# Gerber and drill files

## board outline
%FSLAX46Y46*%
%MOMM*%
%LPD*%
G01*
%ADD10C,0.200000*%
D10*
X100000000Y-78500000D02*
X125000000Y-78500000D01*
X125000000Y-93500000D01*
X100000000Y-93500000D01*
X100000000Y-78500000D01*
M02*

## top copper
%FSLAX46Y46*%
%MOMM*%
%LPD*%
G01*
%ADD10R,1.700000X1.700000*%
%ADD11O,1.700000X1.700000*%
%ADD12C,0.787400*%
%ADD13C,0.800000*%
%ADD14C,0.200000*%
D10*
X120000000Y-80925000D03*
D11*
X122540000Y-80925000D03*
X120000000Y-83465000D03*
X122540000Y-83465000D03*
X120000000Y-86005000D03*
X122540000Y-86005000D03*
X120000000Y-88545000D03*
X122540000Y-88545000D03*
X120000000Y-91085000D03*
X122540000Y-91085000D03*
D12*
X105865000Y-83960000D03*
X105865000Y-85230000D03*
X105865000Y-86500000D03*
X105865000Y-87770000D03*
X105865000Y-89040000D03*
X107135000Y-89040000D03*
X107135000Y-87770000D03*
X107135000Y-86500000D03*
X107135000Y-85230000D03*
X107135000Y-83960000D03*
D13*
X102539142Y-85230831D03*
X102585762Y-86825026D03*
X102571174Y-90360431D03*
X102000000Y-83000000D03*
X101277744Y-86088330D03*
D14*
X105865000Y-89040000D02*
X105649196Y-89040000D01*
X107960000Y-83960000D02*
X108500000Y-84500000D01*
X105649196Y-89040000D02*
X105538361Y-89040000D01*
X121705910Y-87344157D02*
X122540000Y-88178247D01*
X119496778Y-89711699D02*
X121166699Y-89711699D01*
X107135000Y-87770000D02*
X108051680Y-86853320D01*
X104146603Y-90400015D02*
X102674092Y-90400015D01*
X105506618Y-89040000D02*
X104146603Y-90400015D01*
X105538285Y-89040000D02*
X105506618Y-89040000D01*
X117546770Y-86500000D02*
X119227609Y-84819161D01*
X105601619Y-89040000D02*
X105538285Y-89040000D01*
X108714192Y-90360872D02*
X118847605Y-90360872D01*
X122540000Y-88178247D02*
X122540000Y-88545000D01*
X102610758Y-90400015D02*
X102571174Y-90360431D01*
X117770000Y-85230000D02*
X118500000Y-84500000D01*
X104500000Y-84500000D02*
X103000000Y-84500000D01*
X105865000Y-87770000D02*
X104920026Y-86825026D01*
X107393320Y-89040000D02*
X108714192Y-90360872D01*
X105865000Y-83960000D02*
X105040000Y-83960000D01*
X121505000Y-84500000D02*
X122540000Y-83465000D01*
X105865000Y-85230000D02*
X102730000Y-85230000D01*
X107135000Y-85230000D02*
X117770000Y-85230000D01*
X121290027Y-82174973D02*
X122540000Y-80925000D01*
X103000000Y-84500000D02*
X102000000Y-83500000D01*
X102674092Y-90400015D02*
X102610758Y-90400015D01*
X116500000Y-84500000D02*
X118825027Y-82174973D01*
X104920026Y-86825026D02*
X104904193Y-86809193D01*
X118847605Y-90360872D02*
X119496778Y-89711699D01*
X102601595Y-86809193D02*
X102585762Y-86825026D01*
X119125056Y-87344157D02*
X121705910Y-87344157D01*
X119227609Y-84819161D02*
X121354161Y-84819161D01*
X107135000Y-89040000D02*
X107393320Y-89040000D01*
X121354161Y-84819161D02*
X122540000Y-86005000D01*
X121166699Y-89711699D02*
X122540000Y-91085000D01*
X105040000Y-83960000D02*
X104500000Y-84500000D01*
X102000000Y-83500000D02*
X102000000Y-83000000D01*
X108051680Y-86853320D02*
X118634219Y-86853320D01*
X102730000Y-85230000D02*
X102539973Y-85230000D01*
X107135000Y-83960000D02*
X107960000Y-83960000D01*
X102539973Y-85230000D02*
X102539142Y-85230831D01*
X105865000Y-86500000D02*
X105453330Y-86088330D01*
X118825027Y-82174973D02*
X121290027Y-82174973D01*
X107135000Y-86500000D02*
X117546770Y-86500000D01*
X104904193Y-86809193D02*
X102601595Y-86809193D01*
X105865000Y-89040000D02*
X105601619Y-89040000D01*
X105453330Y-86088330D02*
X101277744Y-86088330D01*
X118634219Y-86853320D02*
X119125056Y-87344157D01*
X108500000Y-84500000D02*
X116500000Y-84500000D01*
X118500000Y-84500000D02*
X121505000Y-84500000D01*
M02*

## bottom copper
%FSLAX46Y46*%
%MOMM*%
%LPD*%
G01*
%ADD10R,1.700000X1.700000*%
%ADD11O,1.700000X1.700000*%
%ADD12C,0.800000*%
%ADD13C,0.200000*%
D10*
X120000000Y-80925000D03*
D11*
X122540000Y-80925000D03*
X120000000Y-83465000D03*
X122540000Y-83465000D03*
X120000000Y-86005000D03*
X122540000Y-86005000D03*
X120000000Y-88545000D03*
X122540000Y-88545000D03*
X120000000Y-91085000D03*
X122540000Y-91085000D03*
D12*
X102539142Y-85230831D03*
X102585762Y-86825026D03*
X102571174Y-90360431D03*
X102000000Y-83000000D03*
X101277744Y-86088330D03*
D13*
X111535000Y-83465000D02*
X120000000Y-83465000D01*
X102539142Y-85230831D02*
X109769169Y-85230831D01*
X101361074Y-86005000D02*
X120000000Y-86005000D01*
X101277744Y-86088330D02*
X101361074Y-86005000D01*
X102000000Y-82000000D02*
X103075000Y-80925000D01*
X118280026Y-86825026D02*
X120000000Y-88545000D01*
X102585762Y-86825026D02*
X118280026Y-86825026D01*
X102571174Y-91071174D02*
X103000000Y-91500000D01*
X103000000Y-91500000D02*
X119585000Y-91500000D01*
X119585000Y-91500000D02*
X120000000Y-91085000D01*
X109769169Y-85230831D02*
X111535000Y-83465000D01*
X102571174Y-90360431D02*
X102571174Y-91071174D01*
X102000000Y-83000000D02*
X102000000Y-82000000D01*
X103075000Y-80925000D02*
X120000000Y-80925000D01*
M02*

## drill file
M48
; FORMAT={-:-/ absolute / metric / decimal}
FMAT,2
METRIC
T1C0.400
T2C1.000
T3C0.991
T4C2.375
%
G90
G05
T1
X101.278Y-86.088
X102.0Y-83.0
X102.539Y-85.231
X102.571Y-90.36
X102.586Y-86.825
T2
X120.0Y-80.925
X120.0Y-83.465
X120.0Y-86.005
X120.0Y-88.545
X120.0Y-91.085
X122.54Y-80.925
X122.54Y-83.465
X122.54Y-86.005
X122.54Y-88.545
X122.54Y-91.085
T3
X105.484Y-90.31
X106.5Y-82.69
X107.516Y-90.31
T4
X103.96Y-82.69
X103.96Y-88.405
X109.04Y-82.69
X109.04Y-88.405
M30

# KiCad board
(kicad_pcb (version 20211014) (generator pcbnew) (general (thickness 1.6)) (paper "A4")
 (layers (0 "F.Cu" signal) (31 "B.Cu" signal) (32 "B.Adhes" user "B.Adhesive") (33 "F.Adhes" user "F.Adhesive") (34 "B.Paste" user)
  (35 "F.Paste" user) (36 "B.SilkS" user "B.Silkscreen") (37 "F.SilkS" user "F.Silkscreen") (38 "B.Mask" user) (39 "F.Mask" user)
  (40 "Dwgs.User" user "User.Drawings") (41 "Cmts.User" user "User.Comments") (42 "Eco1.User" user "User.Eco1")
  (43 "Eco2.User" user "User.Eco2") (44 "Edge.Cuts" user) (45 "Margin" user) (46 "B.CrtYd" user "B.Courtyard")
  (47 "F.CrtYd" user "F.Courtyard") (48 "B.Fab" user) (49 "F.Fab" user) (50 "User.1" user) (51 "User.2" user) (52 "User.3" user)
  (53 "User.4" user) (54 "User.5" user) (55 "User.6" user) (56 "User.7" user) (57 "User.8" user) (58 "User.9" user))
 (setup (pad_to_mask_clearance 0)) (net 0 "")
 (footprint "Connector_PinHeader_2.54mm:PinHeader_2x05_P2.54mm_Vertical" (layer "F.Cu") (at 120 80.925)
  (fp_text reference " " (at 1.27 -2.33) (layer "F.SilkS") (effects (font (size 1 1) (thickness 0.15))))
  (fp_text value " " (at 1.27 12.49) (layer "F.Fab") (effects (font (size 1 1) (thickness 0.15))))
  (pad "1" thru_hole rect (at 0 0) (size 1.7 1.7) (drill 1) (layers *.Cu *.Mask))
  (pad "2" thru_hole oval (at 2.54 0) (size 1.7 1.7) (drill 1) (layers *.Cu *.Mask))
  (pad "3" thru_hole oval (at 0 2.54) (size 1.7 1.7) (drill 1) (layers *.Cu *.Mask))
  (pad "4" thru_hole oval (at 2.54 2.54) (size 1.7 1.7) (drill 1) (layers *.Cu *.Mask))
  (pad "5" thru_hole oval (at 0 5.08) (size 1.7 1.7) (drill 1) (layers *.Cu *.Mask))
  (pad "6" thru_hole oval (at 2.54 5.08) (size 1.7 1.7) (drill 1) (layers *.Cu *.Mask))
  (pad "7" thru_hole oval (at 0 7.62) (size 1.7 1.7) (drill 1) (layers *.Cu *.Mask))
  (pad "8" thru_hole oval (at 2.54 7.62) (size 1.7 1.7) (drill 1) (layers *.Cu *.Mask))
  (pad "9" thru_hole oval (at 0 10.16) (size 1.7 1.7) (drill 1) (layers *.Cu *.Mask))
  (pad "10" thru_hole oval (at 2.54 10.16) (size 1.7 1.7) (drill 1) (layers *.Cu *.Mask)))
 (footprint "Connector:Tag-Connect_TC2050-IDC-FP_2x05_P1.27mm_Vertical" (layer "F.Cu") (at 106.5 86.5 -90)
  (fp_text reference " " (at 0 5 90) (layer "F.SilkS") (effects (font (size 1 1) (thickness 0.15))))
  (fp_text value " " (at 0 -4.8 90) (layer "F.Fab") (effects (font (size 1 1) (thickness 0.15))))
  (pad "" np_thru_hole circle (at -3.81 0 270) (size 0.9906 0.9906) (drill 0.9906) (layers *.Cu *.Mask))
  (pad "" np_thru_hole circle (at 3.81 -1.016 270) (size 0.9906 0.9906) (drill 0.9906) (layers *.Cu *.Mask))
  (pad "" np_thru_hole circle (at 1.905 2.54 270) (size 2.3749 2.3749) (drill 2.3749) (layers *.Cu *.Mask))
  (pad "" np_thru_hole circle (at -3.81 2.54 270) (size 2.3749 2.3749) (drill 2.3749) (layers *.Cu *.Mask))
  (pad "" np_thru_hole circle (at -3.81 -2.54 270) (size 2.3749 2.3749) (drill 2.3749) (layers *.Cu *.Mask))
  (pad "" np_thru_hole circle (at 1.905 -2.54 270) (size 2.3749 2.3749) (drill 2.3749) (layers *.Cu *.Mask))
  (pad "" np_thru_hole circle (at 3.81 1.016 270) (size 0.9906 0.9906) (drill 0.9906) (layers *.Cu *.Mask))
  (pad "1" connect circle (at -2.54 0.635 270) (size 0.7874 0.7874) (layers "F.Cu" "F.Mask"))
  (pad "2" connect circle (at -1.27 0.635 270) (size 0.7874 0.7874) (layers "F.Cu" "F.Mask"))
  (pad "3" connect circle (at 0 0.635 270) (size 0.7874 0.7874) (layers "F.Cu" "F.Mask"))
  (pad "4" connect circle (at 1.27 0.635 270) (size 0.7874 0.7874) (layers "F.Cu" "F.Mask"))
  (pad "5" connect circle (at 2.54 0.635 270) (size 0.7874 0.7874) (layers "F.Cu" "F.Mask"))
  (pad "6" connect circle (at 2.54 -0.635 270) (size 0.7874 0.7874) (layers "F.Cu" "F.Mask"))
  (pad "7" connect circle (at 1.27 -0.635 270) (size 0.7874 0.7874) (layers "F.Cu" "F.Mask"))
  (pad "8" connect circle (at 0 -0.635 270) (size 0.7874 0.7874) (layers "F.Cu" "F.Mask"))
  (pad "9" connect circle (at -1.27 -0.635 270) (size 0.7874 0.7874) (layers "F.Cu" "F.Mask"))
  (pad "10" connect circle (at -2.54 -0.635 270) (size 0.7874 0.7874) (layers "F.Cu" "F.Mask")))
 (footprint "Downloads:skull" (layer "B.Cu") (at 114.5 86 180)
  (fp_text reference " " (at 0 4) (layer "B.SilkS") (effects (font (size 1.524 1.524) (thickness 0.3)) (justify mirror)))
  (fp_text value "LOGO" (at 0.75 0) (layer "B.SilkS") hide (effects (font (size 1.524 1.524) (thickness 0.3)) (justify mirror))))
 (gr_rect (start 100 78.5) (end 125 93.5) (layer "Edge.Cuts") (width 0.2) (fill none))
 (segment (start 105.865 89.04) (end 105.649196 89.04) (width 0.2) (layer "F.Cu") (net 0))
 (segment (start 107.96 83.96) (end 108.5 84.5) (width 0.2) (layer "F.Cu") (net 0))
 (segment (start 105.649196 89.04) (end 105.538361 89.04) (width 0.2) (layer "F.Cu") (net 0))
 (segment (start 121.70591 87.344157) (end 122.54 88.178247) (width 0.2) (layer "F.Cu") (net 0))
 (segment (start 119.496778 89.711699) (end 121.166699 89.711699) (width 0.2) (layer "F.Cu") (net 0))
 (segment (start 107.135 87.77) (end 108.05168 86.85332) (width 0.2) (layer "F.Cu") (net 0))
 (segment (start 104.146603 90.400015) (end 102.674092 90.400015) (width 0.2) (layer "F.Cu") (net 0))
 (segment (start 105.506618 89.04) (end 104.146603 90.400015) (width 0.2) (layer "F.Cu") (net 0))
 (segment (start 105.538285 89.04) (end 105.506618 89.04) (width 0.2) (layer "F.Cu") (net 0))
 (segment (start 117.54677 86.5) (end 119.227609 84.819161) (width 0.2) (layer "F.Cu") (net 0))
 (segment (start 105.601619 89.04) (end 105.538285 89.04) (width 0.2) (layer "F.Cu") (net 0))
 (segment (start 108.714192 90.360872) (end 118.847605 90.360872) (width 0.2) (layer "F.Cu") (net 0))
 (segment (start 122.54 88.178247) (end 122.54 88.545) (width 0.2) (layer "F.Cu") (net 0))
 (segment (start 102.610758 90.400015) (end 102.571174 90.360431) (width 0.2) (layer "F.Cu") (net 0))
 (segment (start 117.77 85.23) (end 118.5 84.5) (width 0.2) (layer "F.Cu") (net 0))
 (segment (start 104.5 84.5) (end 103 84.5) (width 0.2) (layer "F.Cu") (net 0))
 (segment (start 105.865 87.77) (end 104.920026 86.825026) (width 0.2) (layer "F.Cu") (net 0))
 (segment (start 107.39332 89.04) (end 108.714192 90.360872) (width 0.2) (layer "F.Cu") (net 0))
 (segment (start 105.865 83.96) (end 105.04 83.96) (width 0.2) (layer "F.Cu") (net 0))
 (segment (start 121.505 84.5) (end 122.54 83.465) (width 0.2) (layer "F.Cu") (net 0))
 (segment (start 105.865 85.23) (end 102.73 85.23) (width 0.2) (layer "F.Cu") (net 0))
 (segment (start 107.135 85.23) (end 117.77 85.23) (width 0.2) (layer "F.Cu") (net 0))
 (segment (start 121.290027 82.174973) (end 122.54 80.925) (width 0.2) (layer "F.Cu") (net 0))
 (segment (start 103 84.5) (end 102 83.5) (width 0.2) (layer "F.Cu") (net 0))
 (segment (start 102.674092 90.400015) (end 102.610758 90.400015) (width 0.2) (layer "F.Cu") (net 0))
 (segment (start 116.5 84.5) (end 118.825027 82.174973) (width 0.2) (layer "F.Cu") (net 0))
 (segment (start 104.920026 86.825026) (end 104.904193 86.809193) (width 0.2) (layer "F.Cu") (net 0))
 (segment (start 118.847605 90.360872) (end 119.496778 89.711699) (width 0.2) (layer "F.Cu") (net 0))
 (segment (start 102.601595 86.809193) (end 102.585762 86.825026) (width 0.2) (layer "F.Cu") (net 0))
 (segment (start 119.125056 87.344157) (end 121.70591 87.344157) (width 0.2) (layer "F.Cu") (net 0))
 (segment (start 119.227609 84.819161) (end 121.354161 84.819161) (width 0.2) (layer "F.Cu") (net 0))
 (segment (start 107.135 89.04) (end 107.39332 89.04) (width 0.2) (layer "F.Cu") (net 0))
 (segment (start 121.354161 84.819161) (end 122.54 86.005) (width 0.2) (layer "F.Cu") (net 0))
 (segment (start 121.166699 89.711699) (end 122.54 91.085) (width 0.2) (layer "F.Cu") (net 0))
 (segment (start 105.04 83.96) (end 104.5 84.5) (width 0.2) (layer "F.Cu") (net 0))
 (segment (start 102 83.5) (end 102 83) (width 0.2) (layer "F.Cu") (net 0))
 (segment (start 108.05168 86.85332) (end 118.634219 86.85332) (width 0.2) (layer "F.Cu") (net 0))
 (segment (start 102.73 85.23) (end 102.539973 85.23) (width 0.2) (layer "F.Cu") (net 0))
 (segment (start 107.135 83.96) (end 107.96 83.96) (width 0.2) (layer "F.Cu") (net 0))
 (segment (start 102.539973 85.23) (end 102.539142 85.230831) (width 0.2) (layer "F.Cu") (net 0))
 (segment (start 105.865 86.5) (end 105.45333 86.08833) (width 0.2) (layer "F.Cu") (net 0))
 (segment (start 118.825027 82.174973) (end 121.290027 82.174973) (width 0.2) (layer "F.Cu") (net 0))
 (segment (start 107.135 86.5) (end 117.54677 86.5) (width 0.2) (layer "F.Cu") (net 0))
 (segment (start 104.904193 86.809193) (end 102.601595 86.809193) (width 0.2) (layer "F.Cu") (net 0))
 (segment (start 105.865 89.04) (end 105.601619 89.04) (width 0.2) (layer "F.Cu") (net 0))
 (segment (start 105.45333 86.08833) (end 101.277744 86.08833) (width 0.2) (layer "F.Cu") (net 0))
 (segment (start 118.634219 86.85332) (end 119.125056 87.344157) (width 0.2) (layer "F.Cu") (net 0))
 (segment (start 108.5 84.5) (end 116.5 84.5) (width 0.2) (layer "F.Cu") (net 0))
 (segment (start 118.5 84.5) (end 121.505 84.5) (width 0.2) (layer "F.Cu") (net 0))
 (via (at 102.539142 85.230831) (size 0.8) (drill 0.4) (layers "F.Cu" "B.Cu") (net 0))
 (via (at 102.585762 86.825026) (size 0.8) (drill 0.4) (layers "F.Cu" "B.Cu") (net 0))
 (via (at 102.571174 90.360431) (size 0.8) (drill 0.4) (layers "F.Cu" "B.Cu") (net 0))
 (via (at 102 83) (size 0.8) (drill 0.4) (layers "F.Cu" "B.Cu") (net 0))
 (via (at 101.277744 86.08833) (size 0.8) (drill 0.4) (layers "F.Cu" "B.Cu") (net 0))
 (segment (start 111.535 83.465) (end 120 83.465) (width 0.2) (layer "B.Cu") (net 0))
 (segment (start 102.539142 85.230831) (end 109.769169 85.230831) (width 0.2) (layer "B.Cu") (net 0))
 (segment (start 101.361074 86.005) (end 120 86.005) (width 0.2) (layer "B.Cu") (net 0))
 (segment (start 101.277744 86.08833) (end 101.361074 86.005) (width 0.2) (layer "B.Cu") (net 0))
 (segment (start 102 82) (end 103.075 80.925) (width 0.2) (layer "B.Cu") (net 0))
 (segment (start 118.280026 86.825026) (end 120 88.545) (width 0.2) (layer "B.Cu") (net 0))
 (segment (start 102.585762 86.825026) (end 118.280026 86.825026) (width 0.2) (layer "B.Cu") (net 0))
 (segment (start 102.571174 91.071174) (end 103 91.5) (width 0.2) (layer "B.Cu") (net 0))
 (segment (start 103 91.5) (end 119.585 91.5) (width 0.2) (layer "B.Cu") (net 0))
 (segment (start 119.585 91.5) (end 120 91.085) (width 0.2) (layer "B.Cu") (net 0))
 (segment (start 109.769169 85.230831) (end 111.535 83.465) (width 0.2) (layer "B.Cu") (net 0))
 (segment (start 102.571174 90.360431) (end 102.571174 91.071174) (width 0.2) (layer "B.Cu") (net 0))
 (segment (start 102 83) (end 102 82) (width 0.2) (layer "B.Cu") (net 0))
 (segment (start 103.075 80.925) (end 120 80.925) (width 0.2) (layer "B.Cu") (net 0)))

